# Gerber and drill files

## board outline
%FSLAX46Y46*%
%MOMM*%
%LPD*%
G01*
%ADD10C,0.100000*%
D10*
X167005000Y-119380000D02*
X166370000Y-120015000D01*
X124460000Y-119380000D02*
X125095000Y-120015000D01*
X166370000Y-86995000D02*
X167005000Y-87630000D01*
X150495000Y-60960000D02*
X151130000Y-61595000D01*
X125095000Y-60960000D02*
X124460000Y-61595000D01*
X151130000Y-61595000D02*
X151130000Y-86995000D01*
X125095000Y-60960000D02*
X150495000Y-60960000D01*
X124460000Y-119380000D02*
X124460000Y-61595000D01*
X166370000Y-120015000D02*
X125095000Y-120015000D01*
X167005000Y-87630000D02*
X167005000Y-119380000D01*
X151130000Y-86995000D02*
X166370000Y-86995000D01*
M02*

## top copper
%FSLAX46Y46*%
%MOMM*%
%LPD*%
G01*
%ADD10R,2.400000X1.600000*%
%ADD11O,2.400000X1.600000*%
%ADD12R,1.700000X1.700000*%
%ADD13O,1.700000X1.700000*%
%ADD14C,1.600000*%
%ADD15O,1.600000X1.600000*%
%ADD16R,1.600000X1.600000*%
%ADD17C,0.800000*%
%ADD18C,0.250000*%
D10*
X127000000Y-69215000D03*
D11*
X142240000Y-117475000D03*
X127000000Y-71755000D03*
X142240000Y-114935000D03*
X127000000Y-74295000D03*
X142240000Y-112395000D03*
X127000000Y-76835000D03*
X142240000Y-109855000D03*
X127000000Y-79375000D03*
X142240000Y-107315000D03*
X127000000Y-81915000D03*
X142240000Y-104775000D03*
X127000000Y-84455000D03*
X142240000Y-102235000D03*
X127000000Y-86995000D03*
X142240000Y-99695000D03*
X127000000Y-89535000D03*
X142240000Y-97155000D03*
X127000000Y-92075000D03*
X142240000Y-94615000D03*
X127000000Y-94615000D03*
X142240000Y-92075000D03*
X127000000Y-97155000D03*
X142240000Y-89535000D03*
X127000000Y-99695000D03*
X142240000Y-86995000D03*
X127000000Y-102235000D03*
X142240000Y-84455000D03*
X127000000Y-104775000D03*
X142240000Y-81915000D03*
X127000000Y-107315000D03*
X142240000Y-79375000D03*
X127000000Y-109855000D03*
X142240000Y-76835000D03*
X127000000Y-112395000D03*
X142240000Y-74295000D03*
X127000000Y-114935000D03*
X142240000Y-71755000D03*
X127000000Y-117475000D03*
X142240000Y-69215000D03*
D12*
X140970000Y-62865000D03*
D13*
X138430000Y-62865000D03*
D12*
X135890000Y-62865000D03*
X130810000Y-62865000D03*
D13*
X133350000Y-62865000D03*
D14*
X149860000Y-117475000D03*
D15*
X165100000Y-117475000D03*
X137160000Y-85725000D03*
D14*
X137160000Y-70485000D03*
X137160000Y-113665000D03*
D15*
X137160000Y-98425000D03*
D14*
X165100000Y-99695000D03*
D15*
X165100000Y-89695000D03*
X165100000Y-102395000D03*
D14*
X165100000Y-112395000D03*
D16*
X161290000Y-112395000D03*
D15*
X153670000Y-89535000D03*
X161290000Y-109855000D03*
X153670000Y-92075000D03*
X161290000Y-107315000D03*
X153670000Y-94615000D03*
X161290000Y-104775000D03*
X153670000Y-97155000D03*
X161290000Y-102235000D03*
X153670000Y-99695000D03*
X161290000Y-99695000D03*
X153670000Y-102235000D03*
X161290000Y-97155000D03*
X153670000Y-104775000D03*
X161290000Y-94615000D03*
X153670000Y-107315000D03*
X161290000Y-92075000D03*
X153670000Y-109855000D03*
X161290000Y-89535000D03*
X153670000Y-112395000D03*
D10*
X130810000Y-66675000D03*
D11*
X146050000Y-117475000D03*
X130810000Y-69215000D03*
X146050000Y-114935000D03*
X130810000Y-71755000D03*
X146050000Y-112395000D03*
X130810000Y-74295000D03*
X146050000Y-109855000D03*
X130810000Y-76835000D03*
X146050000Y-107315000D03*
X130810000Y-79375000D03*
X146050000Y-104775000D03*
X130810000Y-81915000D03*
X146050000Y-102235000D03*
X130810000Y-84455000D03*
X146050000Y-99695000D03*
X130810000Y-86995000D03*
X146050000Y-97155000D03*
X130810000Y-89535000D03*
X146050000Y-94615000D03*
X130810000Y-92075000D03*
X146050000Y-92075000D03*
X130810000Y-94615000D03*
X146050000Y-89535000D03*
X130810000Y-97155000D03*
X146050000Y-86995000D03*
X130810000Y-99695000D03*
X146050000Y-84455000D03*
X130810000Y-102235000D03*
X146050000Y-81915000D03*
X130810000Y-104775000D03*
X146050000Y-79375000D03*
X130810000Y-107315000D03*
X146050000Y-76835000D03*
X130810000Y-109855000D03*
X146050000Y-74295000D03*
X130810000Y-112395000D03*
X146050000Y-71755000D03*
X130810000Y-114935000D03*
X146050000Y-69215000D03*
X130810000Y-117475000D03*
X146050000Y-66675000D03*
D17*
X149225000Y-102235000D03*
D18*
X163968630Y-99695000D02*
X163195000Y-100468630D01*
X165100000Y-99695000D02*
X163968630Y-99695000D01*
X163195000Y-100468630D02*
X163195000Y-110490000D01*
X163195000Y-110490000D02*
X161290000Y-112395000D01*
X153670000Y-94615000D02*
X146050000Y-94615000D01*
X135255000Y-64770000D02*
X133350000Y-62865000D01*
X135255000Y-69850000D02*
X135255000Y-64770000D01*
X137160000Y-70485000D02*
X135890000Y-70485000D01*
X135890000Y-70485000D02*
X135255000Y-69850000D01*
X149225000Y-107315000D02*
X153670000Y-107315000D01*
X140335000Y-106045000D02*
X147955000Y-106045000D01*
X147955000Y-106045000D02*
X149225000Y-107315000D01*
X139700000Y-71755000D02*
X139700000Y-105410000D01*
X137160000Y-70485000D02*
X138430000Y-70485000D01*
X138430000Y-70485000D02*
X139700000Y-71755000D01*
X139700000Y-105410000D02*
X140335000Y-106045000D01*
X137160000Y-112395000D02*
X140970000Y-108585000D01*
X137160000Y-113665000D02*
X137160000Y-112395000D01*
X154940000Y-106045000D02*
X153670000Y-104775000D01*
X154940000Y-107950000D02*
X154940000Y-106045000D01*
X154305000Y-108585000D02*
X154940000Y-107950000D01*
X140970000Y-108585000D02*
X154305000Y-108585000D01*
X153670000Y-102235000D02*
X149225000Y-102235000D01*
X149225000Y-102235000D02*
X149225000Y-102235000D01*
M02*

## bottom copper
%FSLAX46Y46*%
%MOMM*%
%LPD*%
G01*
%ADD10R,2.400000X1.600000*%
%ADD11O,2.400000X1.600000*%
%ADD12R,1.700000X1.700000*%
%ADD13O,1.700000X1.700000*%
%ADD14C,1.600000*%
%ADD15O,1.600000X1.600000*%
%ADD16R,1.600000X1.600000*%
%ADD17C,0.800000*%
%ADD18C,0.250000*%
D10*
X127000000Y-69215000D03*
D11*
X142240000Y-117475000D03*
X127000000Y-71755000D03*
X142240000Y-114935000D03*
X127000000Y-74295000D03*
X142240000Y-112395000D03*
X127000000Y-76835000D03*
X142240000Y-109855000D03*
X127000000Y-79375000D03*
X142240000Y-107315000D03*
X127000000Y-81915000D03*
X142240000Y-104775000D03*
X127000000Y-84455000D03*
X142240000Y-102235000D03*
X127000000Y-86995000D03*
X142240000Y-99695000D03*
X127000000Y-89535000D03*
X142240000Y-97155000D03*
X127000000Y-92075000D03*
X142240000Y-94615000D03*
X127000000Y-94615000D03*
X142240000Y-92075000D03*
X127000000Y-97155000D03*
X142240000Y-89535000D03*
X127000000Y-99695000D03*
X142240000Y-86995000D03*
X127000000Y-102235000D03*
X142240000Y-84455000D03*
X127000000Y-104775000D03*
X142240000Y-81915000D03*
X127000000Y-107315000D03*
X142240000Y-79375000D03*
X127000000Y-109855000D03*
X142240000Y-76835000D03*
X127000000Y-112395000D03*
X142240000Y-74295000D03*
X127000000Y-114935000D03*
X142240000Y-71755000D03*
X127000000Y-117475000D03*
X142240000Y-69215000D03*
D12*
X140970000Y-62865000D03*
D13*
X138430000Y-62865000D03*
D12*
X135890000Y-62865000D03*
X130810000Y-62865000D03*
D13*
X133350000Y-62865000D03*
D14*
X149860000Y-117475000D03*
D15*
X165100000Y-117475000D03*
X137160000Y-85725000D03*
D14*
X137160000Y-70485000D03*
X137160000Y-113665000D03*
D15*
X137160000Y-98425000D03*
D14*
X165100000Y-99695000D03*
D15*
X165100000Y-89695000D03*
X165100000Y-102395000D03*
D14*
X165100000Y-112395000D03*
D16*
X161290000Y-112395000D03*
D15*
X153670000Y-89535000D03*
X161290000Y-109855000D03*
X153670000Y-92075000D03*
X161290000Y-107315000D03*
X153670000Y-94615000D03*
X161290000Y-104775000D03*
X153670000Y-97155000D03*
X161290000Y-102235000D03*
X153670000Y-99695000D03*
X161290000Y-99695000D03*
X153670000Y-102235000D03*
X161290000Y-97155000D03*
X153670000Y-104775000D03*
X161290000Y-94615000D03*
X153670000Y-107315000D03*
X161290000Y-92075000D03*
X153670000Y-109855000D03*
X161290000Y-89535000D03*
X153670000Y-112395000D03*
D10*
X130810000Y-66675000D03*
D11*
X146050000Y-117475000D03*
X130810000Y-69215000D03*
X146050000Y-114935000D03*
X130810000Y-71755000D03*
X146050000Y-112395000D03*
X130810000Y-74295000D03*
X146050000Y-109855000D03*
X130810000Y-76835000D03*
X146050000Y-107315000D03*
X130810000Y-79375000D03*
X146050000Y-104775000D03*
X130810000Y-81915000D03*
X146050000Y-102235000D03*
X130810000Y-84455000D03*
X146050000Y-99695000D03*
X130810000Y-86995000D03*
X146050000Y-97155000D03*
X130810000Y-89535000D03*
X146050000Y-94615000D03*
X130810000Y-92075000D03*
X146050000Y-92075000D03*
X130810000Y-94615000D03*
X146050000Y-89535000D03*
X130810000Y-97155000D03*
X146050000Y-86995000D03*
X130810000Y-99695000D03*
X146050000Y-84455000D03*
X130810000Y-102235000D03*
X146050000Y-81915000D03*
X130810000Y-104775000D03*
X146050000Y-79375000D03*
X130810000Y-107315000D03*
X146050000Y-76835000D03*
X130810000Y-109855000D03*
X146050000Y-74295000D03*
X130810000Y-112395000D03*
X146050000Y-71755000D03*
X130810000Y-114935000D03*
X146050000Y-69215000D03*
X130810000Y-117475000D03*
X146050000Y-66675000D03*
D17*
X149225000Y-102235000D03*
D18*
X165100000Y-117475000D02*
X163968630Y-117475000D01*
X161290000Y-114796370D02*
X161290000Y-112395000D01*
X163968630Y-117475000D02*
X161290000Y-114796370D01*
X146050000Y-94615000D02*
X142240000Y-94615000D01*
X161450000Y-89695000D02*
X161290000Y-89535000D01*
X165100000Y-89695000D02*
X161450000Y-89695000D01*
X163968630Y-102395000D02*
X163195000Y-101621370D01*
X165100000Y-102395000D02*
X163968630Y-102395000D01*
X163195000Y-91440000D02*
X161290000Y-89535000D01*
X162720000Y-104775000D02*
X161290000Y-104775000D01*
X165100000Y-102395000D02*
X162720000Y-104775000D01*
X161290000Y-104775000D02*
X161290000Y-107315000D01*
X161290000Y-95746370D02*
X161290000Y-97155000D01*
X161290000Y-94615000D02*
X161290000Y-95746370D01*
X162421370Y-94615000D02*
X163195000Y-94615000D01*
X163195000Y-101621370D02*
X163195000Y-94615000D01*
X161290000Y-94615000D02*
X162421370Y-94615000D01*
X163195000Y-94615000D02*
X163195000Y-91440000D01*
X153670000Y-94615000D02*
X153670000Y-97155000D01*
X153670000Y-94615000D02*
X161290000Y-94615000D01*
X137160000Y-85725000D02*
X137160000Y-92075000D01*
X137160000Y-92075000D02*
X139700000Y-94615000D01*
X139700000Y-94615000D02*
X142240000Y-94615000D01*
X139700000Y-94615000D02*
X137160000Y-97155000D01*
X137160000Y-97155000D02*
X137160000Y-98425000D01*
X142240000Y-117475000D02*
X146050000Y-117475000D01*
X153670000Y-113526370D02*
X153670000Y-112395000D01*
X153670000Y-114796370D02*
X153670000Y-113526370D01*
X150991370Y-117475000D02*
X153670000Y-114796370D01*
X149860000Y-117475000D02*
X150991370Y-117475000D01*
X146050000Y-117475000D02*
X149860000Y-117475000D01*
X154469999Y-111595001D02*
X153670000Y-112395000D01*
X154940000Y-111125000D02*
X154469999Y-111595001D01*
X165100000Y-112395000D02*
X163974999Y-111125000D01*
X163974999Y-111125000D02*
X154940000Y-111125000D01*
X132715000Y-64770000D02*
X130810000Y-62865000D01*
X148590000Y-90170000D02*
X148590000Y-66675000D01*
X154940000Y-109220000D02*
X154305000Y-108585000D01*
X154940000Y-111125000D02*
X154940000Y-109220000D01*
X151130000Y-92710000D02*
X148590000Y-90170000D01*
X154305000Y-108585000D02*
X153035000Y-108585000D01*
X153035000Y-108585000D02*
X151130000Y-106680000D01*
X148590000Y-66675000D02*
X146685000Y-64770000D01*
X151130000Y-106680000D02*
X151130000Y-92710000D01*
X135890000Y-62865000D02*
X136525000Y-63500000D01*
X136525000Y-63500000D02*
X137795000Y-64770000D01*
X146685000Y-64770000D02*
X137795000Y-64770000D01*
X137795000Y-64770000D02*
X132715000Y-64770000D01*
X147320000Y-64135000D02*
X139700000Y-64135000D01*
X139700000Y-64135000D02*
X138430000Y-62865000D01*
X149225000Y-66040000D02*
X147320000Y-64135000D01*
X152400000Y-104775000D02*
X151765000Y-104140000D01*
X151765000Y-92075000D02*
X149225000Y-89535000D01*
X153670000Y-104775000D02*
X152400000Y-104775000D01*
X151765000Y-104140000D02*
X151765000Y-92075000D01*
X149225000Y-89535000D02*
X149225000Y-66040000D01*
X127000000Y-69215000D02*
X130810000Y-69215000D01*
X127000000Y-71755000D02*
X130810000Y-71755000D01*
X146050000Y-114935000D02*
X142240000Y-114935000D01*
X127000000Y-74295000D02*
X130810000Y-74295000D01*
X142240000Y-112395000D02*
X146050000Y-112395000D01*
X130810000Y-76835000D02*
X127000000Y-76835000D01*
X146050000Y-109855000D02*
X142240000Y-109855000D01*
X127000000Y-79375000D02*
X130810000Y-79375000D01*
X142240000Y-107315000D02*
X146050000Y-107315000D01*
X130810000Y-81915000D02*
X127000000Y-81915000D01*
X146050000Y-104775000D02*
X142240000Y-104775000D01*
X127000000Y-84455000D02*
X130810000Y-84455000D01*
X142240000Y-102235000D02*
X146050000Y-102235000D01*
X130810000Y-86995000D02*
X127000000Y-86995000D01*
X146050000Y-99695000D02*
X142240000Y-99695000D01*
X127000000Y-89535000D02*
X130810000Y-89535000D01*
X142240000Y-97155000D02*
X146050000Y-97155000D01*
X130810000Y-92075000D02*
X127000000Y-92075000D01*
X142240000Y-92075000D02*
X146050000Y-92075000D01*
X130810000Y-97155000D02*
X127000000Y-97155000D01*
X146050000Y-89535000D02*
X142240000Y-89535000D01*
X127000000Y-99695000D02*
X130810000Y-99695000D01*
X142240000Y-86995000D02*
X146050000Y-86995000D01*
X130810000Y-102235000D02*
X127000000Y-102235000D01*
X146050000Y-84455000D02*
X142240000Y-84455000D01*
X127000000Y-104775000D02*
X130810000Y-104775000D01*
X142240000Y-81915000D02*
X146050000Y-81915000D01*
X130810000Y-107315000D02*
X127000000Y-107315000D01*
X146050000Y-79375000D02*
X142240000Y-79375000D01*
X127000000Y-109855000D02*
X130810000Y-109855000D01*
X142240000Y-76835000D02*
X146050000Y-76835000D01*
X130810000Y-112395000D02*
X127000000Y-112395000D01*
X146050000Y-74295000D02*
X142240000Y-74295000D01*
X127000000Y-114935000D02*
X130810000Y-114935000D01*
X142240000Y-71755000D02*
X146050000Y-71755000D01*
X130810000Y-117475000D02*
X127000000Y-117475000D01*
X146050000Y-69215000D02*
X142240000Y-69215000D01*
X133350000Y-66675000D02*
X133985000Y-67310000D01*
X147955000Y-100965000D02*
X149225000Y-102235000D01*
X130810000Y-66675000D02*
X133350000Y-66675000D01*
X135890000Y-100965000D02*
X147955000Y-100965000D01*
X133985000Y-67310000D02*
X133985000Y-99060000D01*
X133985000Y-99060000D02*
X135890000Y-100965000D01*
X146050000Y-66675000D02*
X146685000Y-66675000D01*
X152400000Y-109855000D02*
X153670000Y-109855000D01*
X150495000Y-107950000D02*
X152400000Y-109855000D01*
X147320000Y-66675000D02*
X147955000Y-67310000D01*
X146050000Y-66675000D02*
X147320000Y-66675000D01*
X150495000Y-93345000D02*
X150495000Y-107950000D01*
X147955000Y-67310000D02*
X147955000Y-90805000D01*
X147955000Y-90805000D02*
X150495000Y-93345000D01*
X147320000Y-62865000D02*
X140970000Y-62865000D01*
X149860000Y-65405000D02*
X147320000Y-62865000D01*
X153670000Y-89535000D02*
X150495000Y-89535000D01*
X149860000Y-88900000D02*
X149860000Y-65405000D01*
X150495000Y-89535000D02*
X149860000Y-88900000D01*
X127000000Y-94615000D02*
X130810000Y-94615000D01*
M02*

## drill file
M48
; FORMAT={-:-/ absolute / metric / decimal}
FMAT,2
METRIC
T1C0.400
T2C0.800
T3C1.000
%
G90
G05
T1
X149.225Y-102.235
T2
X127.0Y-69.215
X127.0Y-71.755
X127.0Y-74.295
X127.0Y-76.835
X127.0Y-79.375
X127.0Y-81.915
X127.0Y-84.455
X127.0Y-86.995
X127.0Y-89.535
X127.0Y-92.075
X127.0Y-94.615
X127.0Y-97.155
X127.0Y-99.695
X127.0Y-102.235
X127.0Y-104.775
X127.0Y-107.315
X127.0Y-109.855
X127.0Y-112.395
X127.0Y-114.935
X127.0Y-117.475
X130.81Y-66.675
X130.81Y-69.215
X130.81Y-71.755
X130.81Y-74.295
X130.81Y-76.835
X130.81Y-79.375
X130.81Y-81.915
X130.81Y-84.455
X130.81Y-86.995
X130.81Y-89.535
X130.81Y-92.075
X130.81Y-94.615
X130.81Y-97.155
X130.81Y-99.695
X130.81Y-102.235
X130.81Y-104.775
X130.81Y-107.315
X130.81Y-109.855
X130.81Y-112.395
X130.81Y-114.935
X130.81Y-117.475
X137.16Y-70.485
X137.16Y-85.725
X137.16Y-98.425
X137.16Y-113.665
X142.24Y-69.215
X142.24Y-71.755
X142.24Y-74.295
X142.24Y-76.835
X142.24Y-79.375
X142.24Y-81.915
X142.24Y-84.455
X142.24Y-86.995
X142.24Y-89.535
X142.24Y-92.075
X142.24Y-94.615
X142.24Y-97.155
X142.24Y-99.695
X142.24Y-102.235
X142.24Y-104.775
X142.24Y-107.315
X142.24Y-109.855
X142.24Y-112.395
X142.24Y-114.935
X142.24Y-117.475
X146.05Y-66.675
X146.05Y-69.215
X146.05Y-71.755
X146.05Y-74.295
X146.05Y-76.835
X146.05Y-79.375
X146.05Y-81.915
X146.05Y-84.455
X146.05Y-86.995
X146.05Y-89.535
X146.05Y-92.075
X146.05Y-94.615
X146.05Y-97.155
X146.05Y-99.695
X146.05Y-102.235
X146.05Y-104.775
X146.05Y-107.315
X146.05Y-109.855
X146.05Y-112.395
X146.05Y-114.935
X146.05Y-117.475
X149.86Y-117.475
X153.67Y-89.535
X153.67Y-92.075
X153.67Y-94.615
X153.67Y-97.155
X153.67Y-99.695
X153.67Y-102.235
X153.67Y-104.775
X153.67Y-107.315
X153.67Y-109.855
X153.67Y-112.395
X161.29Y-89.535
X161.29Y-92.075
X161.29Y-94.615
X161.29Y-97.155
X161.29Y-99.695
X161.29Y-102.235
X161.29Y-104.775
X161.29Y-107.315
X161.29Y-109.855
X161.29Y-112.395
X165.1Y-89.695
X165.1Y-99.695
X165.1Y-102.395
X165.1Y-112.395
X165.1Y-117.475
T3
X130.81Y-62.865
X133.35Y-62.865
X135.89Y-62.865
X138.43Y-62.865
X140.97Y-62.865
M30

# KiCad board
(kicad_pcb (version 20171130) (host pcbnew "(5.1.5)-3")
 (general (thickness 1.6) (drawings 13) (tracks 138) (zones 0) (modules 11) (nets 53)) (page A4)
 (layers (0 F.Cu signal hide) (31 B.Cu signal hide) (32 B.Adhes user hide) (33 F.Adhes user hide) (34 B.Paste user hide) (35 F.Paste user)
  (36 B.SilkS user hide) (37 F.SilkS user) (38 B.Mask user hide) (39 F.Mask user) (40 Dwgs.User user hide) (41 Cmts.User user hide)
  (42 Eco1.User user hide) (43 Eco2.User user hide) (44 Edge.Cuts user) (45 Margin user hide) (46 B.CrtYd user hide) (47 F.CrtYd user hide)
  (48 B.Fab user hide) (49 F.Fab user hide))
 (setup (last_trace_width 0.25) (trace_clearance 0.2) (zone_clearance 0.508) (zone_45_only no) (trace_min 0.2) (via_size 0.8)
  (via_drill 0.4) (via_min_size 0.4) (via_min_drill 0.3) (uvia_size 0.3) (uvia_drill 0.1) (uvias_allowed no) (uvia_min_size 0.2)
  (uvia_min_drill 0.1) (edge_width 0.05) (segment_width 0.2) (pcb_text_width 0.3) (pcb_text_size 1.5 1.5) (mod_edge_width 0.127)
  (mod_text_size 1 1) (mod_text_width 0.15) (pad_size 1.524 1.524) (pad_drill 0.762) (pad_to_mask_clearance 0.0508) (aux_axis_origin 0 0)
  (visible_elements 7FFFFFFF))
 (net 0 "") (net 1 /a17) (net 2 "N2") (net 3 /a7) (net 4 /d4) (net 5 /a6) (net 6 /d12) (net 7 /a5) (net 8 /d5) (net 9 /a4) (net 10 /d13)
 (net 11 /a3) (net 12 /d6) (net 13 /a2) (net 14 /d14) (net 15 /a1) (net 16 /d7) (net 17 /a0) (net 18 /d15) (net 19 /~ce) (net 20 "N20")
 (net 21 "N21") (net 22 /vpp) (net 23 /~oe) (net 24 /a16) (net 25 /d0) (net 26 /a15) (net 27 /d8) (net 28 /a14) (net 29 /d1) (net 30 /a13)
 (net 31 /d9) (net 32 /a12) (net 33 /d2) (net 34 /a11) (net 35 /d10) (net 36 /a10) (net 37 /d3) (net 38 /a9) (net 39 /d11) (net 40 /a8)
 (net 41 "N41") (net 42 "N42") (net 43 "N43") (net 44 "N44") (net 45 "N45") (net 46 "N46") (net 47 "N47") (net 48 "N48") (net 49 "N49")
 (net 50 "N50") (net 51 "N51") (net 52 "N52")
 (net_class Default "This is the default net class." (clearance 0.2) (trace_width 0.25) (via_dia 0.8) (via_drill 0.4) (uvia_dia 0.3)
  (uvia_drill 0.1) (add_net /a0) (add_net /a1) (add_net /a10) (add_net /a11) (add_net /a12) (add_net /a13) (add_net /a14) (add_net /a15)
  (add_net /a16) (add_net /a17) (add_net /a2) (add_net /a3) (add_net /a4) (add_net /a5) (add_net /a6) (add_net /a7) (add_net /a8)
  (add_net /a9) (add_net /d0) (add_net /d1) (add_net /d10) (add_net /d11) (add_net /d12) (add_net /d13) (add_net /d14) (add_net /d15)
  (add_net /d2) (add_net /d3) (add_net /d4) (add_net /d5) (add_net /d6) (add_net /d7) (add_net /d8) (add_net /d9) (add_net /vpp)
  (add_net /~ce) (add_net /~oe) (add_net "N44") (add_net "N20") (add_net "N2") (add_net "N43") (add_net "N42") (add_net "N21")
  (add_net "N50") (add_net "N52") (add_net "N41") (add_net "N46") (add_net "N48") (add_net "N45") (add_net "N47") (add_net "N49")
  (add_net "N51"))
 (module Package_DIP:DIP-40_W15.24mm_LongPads (layer F.Cu) (at 127 69.215)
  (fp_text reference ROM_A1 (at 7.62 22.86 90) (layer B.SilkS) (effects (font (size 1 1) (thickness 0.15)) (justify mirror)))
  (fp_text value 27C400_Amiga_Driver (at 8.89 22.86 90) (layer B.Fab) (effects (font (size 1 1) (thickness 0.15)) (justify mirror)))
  (pad 1 thru_hole rect (at 0 0) (size 2.4 1.6) (drill 0.8) (layers *.Cu *.Mask) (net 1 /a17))
  (pad 21 thru_hole oval (at 15.24 48.26) (size 2.4 1.6) (drill 0.8) (layers *.Cu *.Mask) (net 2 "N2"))
  (pad 2 thru_hole oval (at 0 2.54) (size 2.4 1.6) (drill 0.8) (layers *.Cu *.Mask) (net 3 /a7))
  (pad 22 thru_hole oval (at 15.24 45.72) (size 2.4 1.6) (drill 0.8) (layers *.Cu *.Mask) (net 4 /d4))
  (pad 3 thru_hole oval (at 0 5.08) (size 2.4 1.6) (drill 0.8) (layers *.Cu *.Mask) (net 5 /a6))
  (pad 23 thru_hole oval (at 15.24 43.18) (size 2.4 1.6) (drill 0.8) (layers *.Cu *.Mask) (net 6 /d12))
  (pad 4 thru_hole oval (at 0 7.62) (size 2.4 1.6) (drill 0.8) (layers *.Cu *.Mask) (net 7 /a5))
  (pad 24 thru_hole oval (at 15.24 40.64) (size 2.4 1.6) (drill 0.8) (layers *.Cu *.Mask) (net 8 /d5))
  (pad 5 thru_hole oval (at 0 10.16) (size 2.4 1.6) (drill 0.8) (layers *.Cu *.Mask) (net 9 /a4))
  (pad 25 thru_hole oval (at 15.24 38.1) (size 2.4 1.6) (drill 0.8) (layers *.Cu *.Mask) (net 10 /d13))
  (pad 6 thru_hole oval (at 0 12.7) (size 2.4 1.6) (drill 0.8) (layers *.Cu *.Mask) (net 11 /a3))
  (pad 26 thru_hole oval (at 15.24 35.56) (size 2.4 1.6) (drill 0.8) (layers *.Cu *.Mask) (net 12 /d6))
  (pad 7 thru_hole oval (at 0 15.24) (size 2.4 1.6) (drill 0.8) (layers *.Cu *.Mask) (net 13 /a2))
  (pad 27 thru_hole oval (at 15.24 33.02) (size 2.4 1.6) (drill 0.8) (layers *.Cu *.Mask) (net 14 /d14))
  (pad 8 thru_hole oval (at 0 17.78) (size 2.4 1.6) (drill 0.8) (layers *.Cu *.Mask) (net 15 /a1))
  (pad 28 thru_hole oval (at 15.24 30.48) (size 2.4 1.6) (drill 0.8) (layers *.Cu *.Mask) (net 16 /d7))
  (pad 9 thru_hole oval (at 0 20.32) (size 2.4 1.6) (drill 0.8) (layers *.Cu *.Mask) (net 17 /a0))
  (pad 29 thru_hole oval (at 15.24 27.94) (size 2.4 1.6) (drill 0.8) (layers *.Cu *.Mask) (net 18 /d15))
  (pad 10 thru_hole oval (at 0 22.86) (size 2.4 1.6) (drill 0.8) (layers *.Cu *.Mask) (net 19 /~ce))
  (pad 30 thru_hole oval (at 15.24 25.4) (size 2.4 1.6) (drill 0.8) (layers *.Cu *.Mask) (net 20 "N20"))
  (pad 11 thru_hole oval (at 0 25.4) (size 2.4 1.6) (drill 0.8) (layers *.Cu *.Mask) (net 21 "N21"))
  (pad 31 thru_hole oval (at 15.24 22.86) (size 2.4 1.6) (drill 0.8) (layers *.Cu *.Mask) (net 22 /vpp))
  (pad 12 thru_hole oval (at 0 27.94) (size 2.4 1.6) (drill 0.8) (layers *.Cu *.Mask) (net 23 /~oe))
  (pad 32 thru_hole oval (at 15.24 20.32) (size 2.4 1.6) (drill 0.8) (layers *.Cu *.Mask) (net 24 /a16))
  (pad 13 thru_hole oval (at 0 30.48) (size 2.4 1.6) (drill 0.8) (layers *.Cu *.Mask) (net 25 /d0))
  (pad 33 thru_hole oval (at 15.24 17.78) (size 2.4 1.6) (drill 0.8) (layers *.Cu *.Mask) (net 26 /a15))
  (pad 14 thru_hole oval (at 0 33.02) (size 2.4 1.6) (drill 0.8) (layers *.Cu *.Mask) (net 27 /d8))
  (pad 34 thru_hole oval (at 15.24 15.24) (size 2.4 1.6) (drill 0.8) (layers *.Cu *.Mask) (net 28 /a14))
  (pad 15 thru_hole oval (at 0 35.56) (size 2.4 1.6) (drill 0.8) (layers *.Cu *.Mask) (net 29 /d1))
  (pad 35 thru_hole oval (at 15.24 12.7) (size 2.4 1.6) (drill 0.8) (layers *.Cu *.Mask) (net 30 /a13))
  (pad 16 thru_hole oval (at 0 38.1) (size 2.4 1.6) (drill 0.8) (layers *.Cu *.Mask) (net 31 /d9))
  (pad 36 thru_hole oval (at 15.24 10.16) (size 2.4 1.6) (drill 0.8) (layers *.Cu *.Mask) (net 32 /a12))
  (pad 17 thru_hole oval (at 0 40.64) (size 2.4 1.6) (drill 0.8) (layers *.Cu *.Mask) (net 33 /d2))
  (pad 37 thru_hole oval (at 15.24 7.62) (size 2.4 1.6) (drill 0.8) (layers *.Cu *.Mask) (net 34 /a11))
  (pad 18 thru_hole oval (at 0 43.18) (size 2.4 1.6) (drill 0.8) (layers *.Cu *.Mask) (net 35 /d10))
  (pad 38 thru_hole oval (at 15.24 5.08) (size 2.4 1.6) (drill 0.8) (layers *.Cu *.Mask) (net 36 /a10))
  (pad 19 thru_hole oval (at 0 45.72) (size 2.4 1.6) (drill 0.8) (layers *.Cu *.Mask) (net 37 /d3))
  (pad 39 thru_hole oval (at 15.24 2.54) (size 2.4 1.6) (drill 0.8) (layers *.Cu *.Mask) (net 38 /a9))
  (pad 20 thru_hole oval (at 0 48.26) (size 2.4 1.6) (drill 0.8) (layers *.Cu *.Mask) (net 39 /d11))
  (pad 40 thru_hole oval (at 15.24 0) (size 2.4 1.6) (drill 0.8) (layers *.Cu *.Mask) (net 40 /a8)))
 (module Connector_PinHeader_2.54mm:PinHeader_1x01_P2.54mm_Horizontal (layer F.Cu) (at 140.97 62.865 90)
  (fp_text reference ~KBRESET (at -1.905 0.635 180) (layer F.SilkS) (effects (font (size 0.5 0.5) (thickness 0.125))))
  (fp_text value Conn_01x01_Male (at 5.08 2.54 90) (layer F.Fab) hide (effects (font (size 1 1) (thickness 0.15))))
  (pad 1 thru_hole rect (at 0 0 90) (size 1.7 1.7) (drill 1) (layers *.Cu *.Mask) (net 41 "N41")))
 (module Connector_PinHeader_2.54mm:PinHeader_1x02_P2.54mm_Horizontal (layer F.Cu) (at 135.89 62.865 90)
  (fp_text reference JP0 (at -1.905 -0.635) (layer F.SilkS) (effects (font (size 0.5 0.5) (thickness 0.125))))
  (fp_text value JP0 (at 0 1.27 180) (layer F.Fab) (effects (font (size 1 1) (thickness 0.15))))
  (pad 2 thru_hole oval (at 0 2.54 90) (size 1.7 1.7) (drill 1) (layers *.Cu *.Mask) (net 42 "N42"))
  (pad 1 thru_hole rect (at 0 0 90) (size 1.7 1.7) (drill 1) (layers *.Cu *.Mask) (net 2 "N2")))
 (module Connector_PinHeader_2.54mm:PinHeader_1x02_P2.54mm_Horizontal (layer F.Cu) (at 130.81 62.865 90)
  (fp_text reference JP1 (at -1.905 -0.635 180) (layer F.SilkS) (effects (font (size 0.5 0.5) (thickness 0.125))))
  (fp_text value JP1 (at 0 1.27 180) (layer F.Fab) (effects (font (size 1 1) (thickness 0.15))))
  (pad 1 thru_hole rect (at 0 0 90) (size 1.7 1.7) (drill 1) (layers *.Cu *.Mask) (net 2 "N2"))
  (pad 2 thru_hole oval (at 0 2.54 90) (size 1.7 1.7) (drill 1) (layers *.Cu *.Mask) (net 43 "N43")))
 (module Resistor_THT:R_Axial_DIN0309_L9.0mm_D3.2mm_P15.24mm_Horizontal (layer F.Cu) (at 149.86 117.475)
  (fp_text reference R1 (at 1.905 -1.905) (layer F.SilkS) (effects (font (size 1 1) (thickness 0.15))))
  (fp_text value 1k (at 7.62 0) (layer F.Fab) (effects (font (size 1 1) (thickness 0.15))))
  (pad 1 thru_hole circle (at 0 0) (size 1.6 1.6) (drill 0.8) (layers *.Cu *.Mask) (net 2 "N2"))
  (pad 2 thru_hole oval (at 15.24 0) (size 1.6 1.6) (drill 0.8) (layers *.Cu *.Mask) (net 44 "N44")))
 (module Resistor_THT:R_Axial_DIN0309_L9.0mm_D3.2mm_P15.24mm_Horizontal (layer F.Cu) (at 137.16 70.485 270)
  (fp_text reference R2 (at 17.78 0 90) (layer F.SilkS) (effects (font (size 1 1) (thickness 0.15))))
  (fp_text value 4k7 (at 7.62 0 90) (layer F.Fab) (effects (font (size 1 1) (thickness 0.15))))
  (pad 2 thru_hole oval (at 15.24 0 270) (size 1.6 1.6) (drill 0.8) (layers *.Cu *.Mask) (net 20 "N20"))
  (pad 1 thru_hole circle (at 0 0 270) (size 1.6 1.6) (drill 0.8) (layers *.Cu *.Mask) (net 43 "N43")))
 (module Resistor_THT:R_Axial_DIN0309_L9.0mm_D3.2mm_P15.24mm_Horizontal (layer F.Cu) (at 137.16 113.665 90)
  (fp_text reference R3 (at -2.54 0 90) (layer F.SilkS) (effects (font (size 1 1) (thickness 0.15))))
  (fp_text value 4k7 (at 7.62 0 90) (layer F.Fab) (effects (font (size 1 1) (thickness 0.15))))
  (pad 1 thru_hole circle (at 0 0 90) (size 1.6 1.6) (drill 0.8) (layers *.Cu *.Mask) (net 42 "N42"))
  (pad 2 thru_hole oval (at 15.24 0 90) (size 1.6 1.6) (drill 0.8) (layers *.Cu *.Mask) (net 20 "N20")))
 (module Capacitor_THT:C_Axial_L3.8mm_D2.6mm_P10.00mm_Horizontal (layer F.Cu) (at 165.1 99.695 90)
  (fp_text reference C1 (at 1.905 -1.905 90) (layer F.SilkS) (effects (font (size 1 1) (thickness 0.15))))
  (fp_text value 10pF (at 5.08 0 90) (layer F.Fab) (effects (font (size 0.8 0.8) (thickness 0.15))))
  (pad 1 thru_hole circle (at 0 0 90) (size 1.6 1.6) (drill 0.8) (layers *.Cu *.Mask) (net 44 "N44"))
  (pad 2 thru_hole oval (at 10 0 90) (size 1.6 1.6) (drill 0.8) (layers *.Cu *.Mask) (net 20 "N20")))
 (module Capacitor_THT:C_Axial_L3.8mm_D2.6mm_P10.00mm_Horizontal (layer F.Cu) (at 165.1 112.395 90)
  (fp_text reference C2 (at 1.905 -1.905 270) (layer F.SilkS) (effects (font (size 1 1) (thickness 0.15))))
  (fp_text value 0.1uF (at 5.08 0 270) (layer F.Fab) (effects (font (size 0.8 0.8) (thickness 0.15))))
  (pad 2 thru_hole oval (at 10 0 90) (size 1.6 1.6) (drill 0.8) (layers *.Cu *.Mask) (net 20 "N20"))
  (pad 1 thru_hole circle (at 0 0 90) (size 1.6 1.6) (drill 0.8) (layers *.Cu *.Mask) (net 2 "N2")))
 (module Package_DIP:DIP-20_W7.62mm (layer F.Cu) (at 161.29 112.395 180)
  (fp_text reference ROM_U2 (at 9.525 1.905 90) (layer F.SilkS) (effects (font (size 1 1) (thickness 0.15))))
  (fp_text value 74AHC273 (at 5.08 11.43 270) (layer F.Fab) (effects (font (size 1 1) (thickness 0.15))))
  (pad 1 thru_hole rect (at 0 0 180) (size 1.6 1.6) (drill 0.8) (layers *.Cu *.Mask) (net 44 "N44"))
  (pad 11 thru_hole oval (at 7.62 22.86 180) (size 1.6 1.6) (drill 0.8) (layers *.Cu *.Mask) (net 41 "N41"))
  (pad 2 thru_hole oval (at 0 2.54 180) (size 1.6 1.6) (drill 0.8) (layers *.Cu *.Mask) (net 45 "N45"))
  (pad 12 thru_hole oval (at 7.62 20.32 180) (size 1.6 1.6) (drill 0.8) (layers *.Cu *.Mask) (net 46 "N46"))
  (pad 3 thru_hole oval (at 0 5.08 180) (size 1.6 1.6) (drill 0.8) (layers *.Cu *.Mask) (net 20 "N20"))
  (pad 13 thru_hole oval (at 7.62 17.78 180) (size 1.6 1.6) (drill 0.8) (layers *.Cu *.Mask) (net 20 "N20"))
  (pad 4 thru_hole oval (at 0 7.62 180) (size 1.6 1.6) (drill 0.8) (layers *.Cu *.Mask) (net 20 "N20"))
  (pad 14 thru_hole oval (at 7.62 15.24 180) (size 1.6 1.6) (drill 0.8) (layers *.Cu *.Mask) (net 20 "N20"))
  (pad 5 thru_hole oval (at 0 10.16 180) (size 1.6 1.6) (drill 0.8) (layers *.Cu *.Mask) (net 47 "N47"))
  (pad 15 thru_hole oval (at 7.62 12.7 180) (size 1.6 1.6) (drill 0.8) (layers *.Cu *.Mask) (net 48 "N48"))
  (pad 6 thru_hole oval (at 0 12.7 180) (size 1.6 1.6) (drill 0.8) (layers *.Cu *.Mask) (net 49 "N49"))
  (pad 16 thru_hole oval (at 7.62 10.16 180) (size 1.6 1.6) (drill 0.8) (layers *.Cu *.Mask) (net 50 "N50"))
  (pad 7 thru_hole oval (at 0 15.24 180) (size 1.6 1.6) (drill 0.8) (layers *.Cu *.Mask) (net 20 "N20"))
  (pad 17 thru_hole oval (at 7.62 7.62 180) (size 1.6 1.6) (drill 0.8) (layers *.Cu *.Mask) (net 42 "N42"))
  (pad 8 thru_hole oval (at 0 17.78 180) (size 1.6 1.6) (drill 0.8) (layers *.Cu *.Mask) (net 20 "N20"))
  (pad 18 thru_hole oval (at 7.62 5.08 180) (size 1.6 1.6) (drill 0.8) (layers *.Cu *.Mask) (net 43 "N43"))
  (pad 9 thru_hole oval (at 0 20.32 180) (size 1.6 1.6) (drill 0.8) (layers *.Cu *.Mask) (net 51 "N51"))
  (pad 19 thru_hole oval (at 7.62 2.54 180) (size 1.6 1.6) (drill 0.8) (layers *.Cu *.Mask) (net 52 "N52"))
  (pad 10 thru_hole oval (at 0 22.86 180) (size 1.6 1.6) (drill 0.8) (layers *.Cu *.Mask) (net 20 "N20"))
  (pad 20 thru_hole oval (at 7.62 0 180) (size 1.6 1.6) (drill 0.8) (layers *.Cu *.Mask) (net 2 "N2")))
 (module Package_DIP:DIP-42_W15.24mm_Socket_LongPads (layer F.Cu) (at 130.81 66.675)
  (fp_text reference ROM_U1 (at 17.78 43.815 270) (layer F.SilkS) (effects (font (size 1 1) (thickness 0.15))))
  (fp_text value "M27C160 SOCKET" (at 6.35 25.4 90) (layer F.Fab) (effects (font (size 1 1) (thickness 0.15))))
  (pad 1 thru_hole rect (at 0 0) (size 2.4 1.6) (drill 0.8) (layers *.Cu *.Mask) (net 50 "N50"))
  (pad 22 thru_hole oval (at 15.24 50.8) (size 2.4 1.6) (drill 0.8) (layers *.Cu *.Mask) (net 2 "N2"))
  (pad 2 thru_hole oval (at 0 2.54) (size 2.4 1.6) (drill 0.8) (layers *.Cu *.Mask) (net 1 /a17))
  (pad 23 thru_hole oval (at 15.24 48.26) (size 2.4 1.6) (drill 0.8) (layers *.Cu *.Mask) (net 4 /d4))
  (pad 3 thru_hole oval (at 0 5.08) (size 2.4 1.6) (drill 0.8) (layers *.Cu *.Mask) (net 3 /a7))
  (pad 24 thru_hole oval (at 15.24 45.72) (size 2.4 1.6) (drill 0.8) (layers *.Cu *.Mask) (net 6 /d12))
  (pad 4 thru_hole oval (at 0 7.62) (size 2.4 1.6) (drill 0.8) (layers *.Cu *.Mask) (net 5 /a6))
  (pad 25 thru_hole oval (at 15.24 43.18) (size 2.4 1.6) (drill 0.8) (layers *.Cu *.Mask) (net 8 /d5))
  (pad 5 thru_hole oval (at 0 10.16) (size 2.4 1.6) (drill 0.8) (layers *.Cu *.Mask) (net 7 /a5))
  (pad 26 thru_hole oval (at 15.24 40.64) (size 2.4 1.6) (drill 0.8) (layers *.Cu *.Mask) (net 10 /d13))
  (pad 6 thru_hole oval (at 0 12.7) (size 2.4 1.6) (drill 0.8) (layers *.Cu *.Mask) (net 9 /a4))
  (pad 27 thru_hole oval (at 15.24 38.1) (size 2.4 1.6) (drill 0.8) (layers *.Cu *.Mask) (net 12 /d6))
  (pad 7 thru_hole oval (at 0 15.24) (size 2.4 1.6) (drill 0.8) (layers *.Cu *.Mask) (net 11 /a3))
  (pad 28 thru_hole oval (at 15.24 35.56) (size 2.4 1.6) (drill 0.8) (layers *.Cu *.Mask) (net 14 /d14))
  (pad 8 thru_hole oval (at 0 17.78) (size 2.4 1.6) (drill 0.8) (layers *.Cu *.Mask) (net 13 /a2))
  (pad 29 thru_hole oval (at 15.24 33.02) (size 2.4 1.6) (drill 0.8) (layers *.Cu *.Mask) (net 16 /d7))
  (pad 9 thru_hole oval (at 0 20.32) (size 2.4 1.6) (drill 0.8) (layers *.Cu *.Mask) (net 15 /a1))
  (pad 30 thru_hole oval (at 15.24 30.48) (size 2.4 1.6) (drill 0.8) (layers *.Cu *.Mask) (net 18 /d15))
  (pad 10 thru_hole oval (at 0 22.86) (size 2.4 1.6) (drill 0.8) (layers *.Cu *.Mask) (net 17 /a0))
  (pad 31 thru_hole oval (at 15.24 27.94) (size 2.4 1.6) (drill 0.8) (layers *.Cu *.Mask) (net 20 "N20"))
  (pad 11 thru_hole oval (at 0 25.4) (size 2.4 1.6) (drill 0.8) (layers *.Cu *.Mask) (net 19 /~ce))
  (pad 32 thru_hole oval (at 15.24 25.4) (size 2.4 1.6) (drill 0.8) (layers *.Cu *.Mask) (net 22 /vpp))
  (pad 12 thru_hole oval (at 0 27.94) (size 2.4 1.6) (drill 0.8) (layers *.Cu *.Mask) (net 21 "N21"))
  (pad 33 thru_hole oval (at 15.24 22.86) (size 2.4 1.6) (drill 0.8) (layers *.Cu *.Mask) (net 24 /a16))
  (pad 13 thru_hole oval (at 0 30.48) (size 2.4 1.6) (drill 0.8) (layers *.Cu *.Mask) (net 23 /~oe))
  (pad 34 thru_hole oval (at 15.24 20.32) (size 2.4 1.6) (drill 0.8) (layers *.Cu *.Mask) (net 26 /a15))
  (pad 14 thru_hole oval (at 0 33.02) (size 2.4 1.6) (drill 0.8) (layers *.Cu *.Mask) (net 25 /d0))
  (pad 35 thru_hole oval (at 15.24 17.78) (size 2.4 1.6) (drill 0.8) (layers *.Cu *.Mask) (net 28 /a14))
  (pad 15 thru_hole oval (at 0 35.56) (size 2.4 1.6) (drill 0.8) (layers *.Cu *.Mask) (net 27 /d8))
  (pad 36 thru_hole oval (at 15.24 15.24) (size 2.4 1.6) (drill 0.8) (layers *.Cu *.Mask) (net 30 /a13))
  (pad 16 thru_hole oval (at 0 38.1) (size 2.4 1.6) (drill 0.8) (layers *.Cu *.Mask) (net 29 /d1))
  (pad 37 thru_hole oval (at 15.24 12.7) (size 2.4 1.6) (drill 0.8) (layers *.Cu *.Mask) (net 32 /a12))
  (pad 17 thru_hole oval (at 0 40.64) (size 2.4 1.6) (drill 0.8) (layers *.Cu *.Mask) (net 31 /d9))
  (pad 38 thru_hole oval (at 15.24 10.16) (size 2.4 1.6) (drill 0.8) (layers *.Cu *.Mask) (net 34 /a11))
  (pad 18 thru_hole oval (at 0 43.18) (size 2.4 1.6) (drill 0.8) (layers *.Cu *.Mask) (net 33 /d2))
  (pad 39 thru_hole oval (at 15.24 7.62) (size 2.4 1.6) (drill 0.8) (layers *.Cu *.Mask) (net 36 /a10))
  (pad 19 thru_hole oval (at 0 45.72) (size 2.4 1.6) (drill 0.8) (layers *.Cu *.Mask) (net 35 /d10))
  (pad 40 thru_hole oval (at 15.24 5.08) (size 2.4 1.6) (drill 0.8) (layers *.Cu *.Mask) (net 38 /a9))
  (pad 20 thru_hole oval (at 0 48.26) (size 2.4 1.6) (drill 0.8) (layers *.Cu *.Mask) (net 37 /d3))
  (pad 41 thru_hole oval (at 15.24 2.54) (size 2.4 1.6) (drill 0.8) (layers *.Cu *.Mask) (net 40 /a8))
  (pad 21 thru_hole oval (at 0 50.8) (size 2.4 1.6) (drill 0.8) (layers *.Cu *.Mask) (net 39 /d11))
  (pad 42 thru_hole oval (at 15.24 0) (size 2.4 1.6) (drill 0.8) (layers *.Cu *.Mask) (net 52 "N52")))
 (gr_line (start 167.005 119.38) (end 166.37 120.015) (layer Edge.Cuts) (width 0.1))
 (gr_line (start 124.46 119.38) (end 125.095 120.015) (layer Edge.Cuts) (width 0.1))
 (gr_line (start 166.37 86.995) (end 167.005 87.63) (layer Edge.Cuts) (width 0.1))
 (gr_line (start 150.495 60.96) (end 151.13 61.595) (layer Edge.Cuts) (width 0.1))
 (gr_line (start 125.095 60.96) (end 124.46 61.595) (layer Edge.Cuts) (width 0.1))
 (gr_line (start 151.13 61.595) (end 151.13 86.995) (layer Edge.Cuts) (width 0.1))
 (gr_line (start 125.095 60.96) (end 150.495 60.96) (layer Edge.Cuts) (width 0.1))
 (gr_line (start 124.46 119.38) (end 124.46 61.595) (layer Edge.Cuts) (width 0.1))
 (gr_line (start 166.37 120.015) (end 125.095 120.015) (layer Edge.Cuts) (width 0.1))
 (gr_line (start 167.005 87.63) (end 167.005 119.38) (layer Edge.Cuts) (width 0.1))
 (gr_line (start 151.13 86.995) (end 166.37 86.995) (layer Edge.Cuts) (width 0.1))
 (segment (start 165.1 117.475) (end 163.96863 117.475) (width 0.25) (layer B.Cu) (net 44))
 (segment (start 161.29 114.79637) (end 161.29 112.395) (width 0.25) (layer B.Cu) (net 44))
 (segment (start 163.96863 117.475) (end 161.29 114.79637) (width 0.25) (layer B.Cu) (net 44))
 (segment (start 163.96863 99.695) (end 163.195 100.46863) (width 0.25) (layer F.Cu) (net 44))
 (segment (start 165.1 99.695) (end 163.96863 99.695) (width 0.25) (layer F.Cu) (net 44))
 (segment (start 163.195 100.46863) (end 163.195 110.49) (width 0.25) (layer F.Cu) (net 44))
 (segment (start 163.195 110.49) (end 161.29 112.395) (width 0.25) (layer F.Cu) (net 44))
 (segment (start 146.05 94.615) (end 142.24 94.615) (width 0.25) (layer B.Cu) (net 20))
 (segment (start 161.45 89.695) (end 161.29 89.535) (width 0.25) (layer B.Cu) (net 20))
 (segment (start 165.1 89.695) (end 161.45 89.695) (width 0.25) (layer B.Cu) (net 20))
 (segment (start 163.96863 102.395) (end 163.195 101.62137) (width 0.25) (layer B.Cu) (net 20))
 (segment (start 165.1 102.395) (end 163.96863 102.395) (width 0.25) (layer B.Cu) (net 20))
 (segment (start 163.195 91.44) (end 161.29 89.535) (width 0.25) (layer B.Cu) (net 20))
 (segment (start 162.72 104.775) (end 161.29 104.775) (width 0.25) (layer B.Cu) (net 20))
 (segment (start 165.1 102.395) (end 162.72 104.775) (width 0.25) (layer B.Cu) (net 20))
 (segment (start 161.29 104.775) (end 161.29 107.315) (width 0.25) (layer B.Cu) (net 20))
 (segment (start 161.29 95.74637) (end 161.29 97.155) (width 0.25) (layer B.Cu) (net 20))
 (segment (start 161.29 94.615) (end 161.29 95.74637) (width 0.25) (layer B.Cu) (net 20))
 (segment (start 162.42137 94.615) (end 163.195 94.615) (width 0.25) (layer B.Cu) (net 20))
 (segment (start 163.195 101.62137) (end 163.195 94.615) (width 0.25) (layer B.Cu) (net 20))
 (segment (start 161.29 94.615) (end 162.42137 94.615) (width 0.25) (layer B.Cu) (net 20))
 (segment (start 163.195 94.615) (end 163.195 91.44) (width 0.25) (layer B.Cu) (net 20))
 (segment (start 153.67 94.615) (end 153.67 97.155) (width 0.25) (layer B.Cu) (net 20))
 (segment (start 153.67 94.615) (end 161.29 94.615) (width 0.25) (layer B.Cu) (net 20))
 (segment (start 153.67 94.615) (end 146.05 94.615) (width 0.25) (layer F.Cu) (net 20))
 (segment (start 137.16 85.725) (end 137.16 92.075) (width 0.25) (layer B.Cu) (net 20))
 (segment (start 137.16 92.075) (end 139.7 94.615) (width 0.25) (layer B.Cu) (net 20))
 (segment (start 139.7 94.615) (end 142.24 94.615) (width 0.25) (layer B.Cu) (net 20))
 (segment (start 139.7 94.615) (end 137.16 97.155) (width 0.25) (layer B.Cu) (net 20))
 (segment (start 137.16 97.155) (end 137.16 98.425) (width 0.25) (layer B.Cu) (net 20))
 (segment (start 142.24 117.475) (end 146.05 117.475) (width 0.25) (layer B.Cu) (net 2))
 (segment (start 153.67 113.52637) (end 153.67 112.395) (width 0.25) (layer B.Cu) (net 2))
 (segment (start 153.67 114.79637) (end 153.67 113.52637) (width 0.25) (layer B.Cu) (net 2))
 (segment (start 150.99137 117.475) (end 153.67 114.79637) (width 0.25) (layer B.Cu) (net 2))
 (segment (start 149.86 117.475) (end 150.99137 117.475) (width 0.25) (layer B.Cu) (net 2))
 (segment (start 146.05 117.475) (end 149.86 117.475) (width 0.25) (layer B.Cu) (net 2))
 (segment (start 154.469999 111.595001) (end 153.67 112.395) (width 0.25) (layer B.Cu) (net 2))
 (segment (start 154.94 111.125) (end 154.469999 111.595001) (width 0.25) (layer B.Cu) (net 2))
 (segment (start 165.1 112.395) (end 163.974999 111.125) (width 0.25) (layer B.Cu) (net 2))
 (segment (start 163.974999 111.125) (end 154.94 111.125) (width 0.25) (layer B.Cu) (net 2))
 (segment (start 132.715 64.77) (end 130.81 62.865) (width 0.25) (layer B.Cu) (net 2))
 (segment (start 148.59 90.17) (end 148.59 66.675) (width 0.25) (layer B.Cu) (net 2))
 (segment (start 154.94 109.22) (end 154.305 108.585) (width 0.25) (layer B.Cu) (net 2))
 (segment (start 154.94 111.125) (end 154.94 109.22) (width 0.25) (layer B.Cu) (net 2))
 (segment (start 151.13 92.71) (end 148.59 90.17) (width 0.25) (layer B.Cu) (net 2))
 (segment (start 154.305 108.585) (end 153.035 108.585) (width 0.25) (layer B.Cu) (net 2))
 (segment (start 153.035 108.585) (end 151.13 106.68) (width 0.25) (layer B.Cu) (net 2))
 (segment (start 148.59 66.675) (end 146.685 64.77) (width 0.25) (layer B.Cu) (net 2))
 (segment (start 151.13 106.68) (end 151.13 92.71) (width 0.25) (layer B.Cu) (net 2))
 (segment (start 135.89 62.865) (end 136.525 63.5) (width 0.25) (layer B.Cu) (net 2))
 (segment (start 136.525 63.5) (end 137.795 64.77) (width 0.25) (layer B.Cu) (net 2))
 (segment (start 146.685 64.77) (end 137.795 64.77) (width 0.25) (layer B.Cu) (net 2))
 (segment (start 137.795 64.77) (end 132.715 64.77) (width 0.25) (layer B.Cu) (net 2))
 (segment (start 135.255 64.77) (end 133.35 62.865) (width 0.25) (layer F.Cu) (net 43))
 (segment (start 135.255 69.85) (end 135.255 64.77) (width 0.25) (layer F.Cu) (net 43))
 (segment (start 137.16 70.485) (end 135.89 70.485) (width 0.25) (layer F.Cu) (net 43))
 (segment (start 135.89 70.485) (end 135.255 69.85) (width 0.25) (layer F.Cu) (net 43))
 (segment (start 149.225 107.315) (end 153.67 107.315) (width 0.25) (layer F.Cu) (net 43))
 (segment (start 140.335 106.045) (end 147.955 106.045) (width 0.25) (layer F.Cu) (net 43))
 (segment (start 147.955 106.045) (end 149.225 107.315) (width 0.25) (layer F.Cu) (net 43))
 (segment (start 139.7 71.755) (end 139.7 105.41) (width 0.25) (layer F.Cu) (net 43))
 (segment (start 137.16 70.485) (end 138.43 70.485) (width 0.25) (layer F.Cu) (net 43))
 (segment (start 138.43 70.485) (end 139.7 71.755) (width 0.25) (layer F.Cu) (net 43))
 (segment (start 139.7 105.41) (end 140.335 106.045) (width 0.25) (layer F.Cu) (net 43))
 (segment (start 137.16 112.395) (end 140.97 108.585) (width 0.25) (layer F.Cu) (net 42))
 (segment (start 137.16 113.665) (end 137.16 112.395) (width 0.25) (layer F.Cu) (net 42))
 (segment (start 154.94 106.045) (end 153.67 104.775) (width 0.25) (layer F.Cu) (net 42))
 (segment (start 154.94 107.95) (end 154.94 106.045) (width 0.25) (layer F.Cu) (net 42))
 (segment (start 154.305 108.585) (end 154.94 107.95) (width 0.25) (layer F.Cu) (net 42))
 (segment (start 140.97 108.585) (end 154.305 108.585) (width 0.25) (layer F.Cu) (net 42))
 (segment (start 147.32 64.135) (end 139.7 64.135) (width 0.25) (layer B.Cu) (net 42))
 (segment (start 139.7 64.135) (end 138.43 62.865) (width 0.25) (layer B.Cu) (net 42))
 (segment (start 149.225 66.04) (end 147.32 64.135) (width 0.25) (layer B.Cu) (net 42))
 (segment (start 152.4 104.775) (end 151.765 104.14) (width 0.25) (layer B.Cu) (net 42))
 (segment (start 151.765 92.075) (end 149.225 89.535) (width 0.25) (layer B.Cu) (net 42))
 (segment (start 153.67 104.775) (end 152.4 104.775) (width 0.25) (layer B.Cu) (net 42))
 (segment (start 151.765 104.14) (end 151.765 92.075) (width 0.25) (layer B.Cu) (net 42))
 (segment (start 149.225 89.535) (end 149.225 66.04) (width 0.25) (layer B.Cu) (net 42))
 (segment (start 127 69.215) (end 130.81 69.215) (width 0.25) (layer B.Cu) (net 1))
 (segment (start 127 71.755) (end 130.81 71.755) (width 0.25) (layer B.Cu) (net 3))
 (segment (start 146.05 114.935) (end 142.24 114.935) (width 0.25) (layer B.Cu) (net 4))
 (segment (start 127 74.295) (end 130.81 74.295) (width 0.25) (layer B.Cu) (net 5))
 (segment (start 142.24 112.395) (end 146.05 112.395) (width 0.25) (layer B.Cu) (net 6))
 (segment (start 130.81 76.835) (end 127 76.835) (width 0.25) (layer B.Cu) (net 7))
 (segment (start 146.05 109.855) (end 142.24 109.855) (width 0.25) (layer B.Cu) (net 8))
 (segment (start 127 79.375) (end 130.81 79.375) (width 0.25) (layer B.Cu) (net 9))
 (segment (start 142.24 107.315) (end 146.05 107.315) (width 0.25) (layer B.Cu) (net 10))
 (segment (start 130.81 81.915) (end 127 81.915) (width 0.25) (layer B.Cu) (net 11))
 (segment (start 146.05 104.775) (end 142.24 104.775) (width 0.25) (layer B.Cu) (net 12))
 (segment (start 127 84.455) (end 130.81 84.455) (width 0.25) (layer B.Cu) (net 13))
 (segment (start 142.24 102.235) (end 146.05 102.235) (width 0.25) (layer B.Cu) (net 14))
 (segment (start 130.81 86.995) (end 127 86.995) (width 0.25) (layer B.Cu) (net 15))
 (segment (start 146.05 99.695) (end 142.24 99.695) (width 0.25) (layer B.Cu) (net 16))
 (segment (start 127 89.535) (end 130.81 89.535) (width 0.25) (layer B.Cu) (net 17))
 (segment (start 142.24 97.155) (end 146.05 97.155) (width 0.25) (layer B.Cu) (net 18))
 (segment (start 130.81 92.075) (end 127 92.075) (width 0.25) (layer B.Cu) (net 19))
 (segment (start 142.24 92.075) (end 146.05 92.075) (width 0.25) (layer B.Cu) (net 22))
 (segment (start 130.81 97.155) (end 127 97.155) (width 0.25) (layer B.Cu) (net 23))
 (segment (start 146.05 89.535) (end 142.24 89.535) (width 0.25) (layer B.Cu) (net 24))
 (segment (start 127 99.695) (end 130.81 99.695) (width 0.25) (layer B.Cu) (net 25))
 (segment (start 142.24 86.995) (end 146.05 86.995) (width 0.25) (layer B.Cu) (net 26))
 (segment (start 130.81 102.235) (end 127 102.235) (width 0.25) (layer B.Cu) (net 27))
 (segment (start 146.05 84.455) (end 142.24 84.455) (width 0.25) (layer B.Cu) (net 28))
 (segment (start 127 104.775) (end 130.81 104.775) (width 0.25) (layer B.Cu) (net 29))
 (segment (start 142.24 81.915) (end 146.05 81.915) (width 0.25) (layer B.Cu) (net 30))
 (segment (start 130.81 107.315) (end 127 107.315) (width 0.25) (layer B.Cu) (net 31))
 (segment (start 146.05 79.375) (end 142.24 79.375) (width 0.25) (layer B.Cu) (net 32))
 (segment (start 127 109.855) (end 130.81 109.855) (width 0.25) (layer B.Cu) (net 33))
 (segment (start 142.24 76.835) (end 146.05 76.835) (width 0.25) (layer B.Cu) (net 34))
 (segment (start 130.81 112.395) (end 127 112.395) (width 0.25) (layer B.Cu) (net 35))
 (segment (start 146.05 74.295) (end 142.24 74.295) (width 0.25) (layer B.Cu) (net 36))
 (segment (start 127 114.935) (end 130.81 114.935) (width 0.25) (layer B.Cu) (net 37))
 (segment (start 142.24 71.755) (end 146.05 71.755) (width 0.25) (layer B.Cu) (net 38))
 (segment (start 130.81 117.475) (end 127 117.475) (width 0.25) (layer B.Cu) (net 39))
 (segment (start 146.05 69.215) (end 142.24 69.215) (width 0.25) (layer B.Cu) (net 40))
 (segment (start 133.35 66.675) (end 133.985 67.31) (width 0.25) (layer B.Cu) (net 50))
 (segment (start 147.955 100.965) (end 149.225 102.235) (width 0.25) (layer B.Cu) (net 50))
 (segment (start 130.81 66.675) (end 133.35 66.675) (width 0.25) (layer B.Cu) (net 50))
 (segment (start 135.89 100.965) (end 147.955 100.965) (width 0.25) (layer B.Cu) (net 50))
 (segment (start 133.985 67.31) (end 133.985 99.06) (width 0.25) (layer B.Cu) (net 50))
 (segment (start 133.985 99.06) (end 135.89 100.965) (width 0.25) (layer B.Cu) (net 50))
 (segment (start 153.67 102.235) (end 149.225 102.235) (width 0.25) (layer F.Cu) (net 50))
 (segment (start 149.225 102.235) (end 149.225 102.235) (width 0.25) (layer F.Cu) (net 50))
 (via (at 149.225 102.235) (size 0.8) (drill 0.4) (layers F.Cu B.Cu) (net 50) (status 1000000))
 (segment (start 146.05 66.675) (end 146.685 66.675) (width 0.25) (layer B.Cu) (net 52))
 (segment (start 152.4 109.855) (end 153.67 109.855) (width 0.25) (layer B.Cu) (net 52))
 (segment (start 150.495 107.95) (end 152.4 109.855) (width 0.25) (layer B.Cu) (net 52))
 (segment (start 147.32 66.675) (end 147.955 67.31) (width 0.25) (layer B.Cu) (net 52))
 (segment (start 146.05 66.675) (end 147.32 66.675) (width 0.25) (layer B.Cu) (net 52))
 (segment (start 150.495 93.345) (end 150.495 107.95) (width 0.25) (layer B.Cu) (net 52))
 (segment (start 147.955 67.31) (end 147.955 90.805) (width 0.25) (layer B.Cu) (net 52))
 (segment (start 147.955 90.805) (end 150.495 93.345) (width 0.25) (layer B.Cu) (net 52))
 (segment (start 147.32 62.865) (end 140.97 62.865) (width 0.25) (layer B.Cu) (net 41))
 (segment (start 149.86 65.405) (end 147.32 62.865) (width 0.25) (layer B.Cu) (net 41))
 (segment (start 153.67 89.535) (end 150.495 89.535) (width 0.25) (layer B.Cu) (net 41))
 (segment (start 149.86 88.9) (end 149.86 65.405) (width 0.25) (layer B.Cu) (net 41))
 (segment (start 150.495 89.535) (end 149.86 88.9) (width 0.25) (layer B.Cu) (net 41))
 (segment (start 127 94.615) (end 130.81 94.615) (width 0.25) (layer B.Cu) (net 21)))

